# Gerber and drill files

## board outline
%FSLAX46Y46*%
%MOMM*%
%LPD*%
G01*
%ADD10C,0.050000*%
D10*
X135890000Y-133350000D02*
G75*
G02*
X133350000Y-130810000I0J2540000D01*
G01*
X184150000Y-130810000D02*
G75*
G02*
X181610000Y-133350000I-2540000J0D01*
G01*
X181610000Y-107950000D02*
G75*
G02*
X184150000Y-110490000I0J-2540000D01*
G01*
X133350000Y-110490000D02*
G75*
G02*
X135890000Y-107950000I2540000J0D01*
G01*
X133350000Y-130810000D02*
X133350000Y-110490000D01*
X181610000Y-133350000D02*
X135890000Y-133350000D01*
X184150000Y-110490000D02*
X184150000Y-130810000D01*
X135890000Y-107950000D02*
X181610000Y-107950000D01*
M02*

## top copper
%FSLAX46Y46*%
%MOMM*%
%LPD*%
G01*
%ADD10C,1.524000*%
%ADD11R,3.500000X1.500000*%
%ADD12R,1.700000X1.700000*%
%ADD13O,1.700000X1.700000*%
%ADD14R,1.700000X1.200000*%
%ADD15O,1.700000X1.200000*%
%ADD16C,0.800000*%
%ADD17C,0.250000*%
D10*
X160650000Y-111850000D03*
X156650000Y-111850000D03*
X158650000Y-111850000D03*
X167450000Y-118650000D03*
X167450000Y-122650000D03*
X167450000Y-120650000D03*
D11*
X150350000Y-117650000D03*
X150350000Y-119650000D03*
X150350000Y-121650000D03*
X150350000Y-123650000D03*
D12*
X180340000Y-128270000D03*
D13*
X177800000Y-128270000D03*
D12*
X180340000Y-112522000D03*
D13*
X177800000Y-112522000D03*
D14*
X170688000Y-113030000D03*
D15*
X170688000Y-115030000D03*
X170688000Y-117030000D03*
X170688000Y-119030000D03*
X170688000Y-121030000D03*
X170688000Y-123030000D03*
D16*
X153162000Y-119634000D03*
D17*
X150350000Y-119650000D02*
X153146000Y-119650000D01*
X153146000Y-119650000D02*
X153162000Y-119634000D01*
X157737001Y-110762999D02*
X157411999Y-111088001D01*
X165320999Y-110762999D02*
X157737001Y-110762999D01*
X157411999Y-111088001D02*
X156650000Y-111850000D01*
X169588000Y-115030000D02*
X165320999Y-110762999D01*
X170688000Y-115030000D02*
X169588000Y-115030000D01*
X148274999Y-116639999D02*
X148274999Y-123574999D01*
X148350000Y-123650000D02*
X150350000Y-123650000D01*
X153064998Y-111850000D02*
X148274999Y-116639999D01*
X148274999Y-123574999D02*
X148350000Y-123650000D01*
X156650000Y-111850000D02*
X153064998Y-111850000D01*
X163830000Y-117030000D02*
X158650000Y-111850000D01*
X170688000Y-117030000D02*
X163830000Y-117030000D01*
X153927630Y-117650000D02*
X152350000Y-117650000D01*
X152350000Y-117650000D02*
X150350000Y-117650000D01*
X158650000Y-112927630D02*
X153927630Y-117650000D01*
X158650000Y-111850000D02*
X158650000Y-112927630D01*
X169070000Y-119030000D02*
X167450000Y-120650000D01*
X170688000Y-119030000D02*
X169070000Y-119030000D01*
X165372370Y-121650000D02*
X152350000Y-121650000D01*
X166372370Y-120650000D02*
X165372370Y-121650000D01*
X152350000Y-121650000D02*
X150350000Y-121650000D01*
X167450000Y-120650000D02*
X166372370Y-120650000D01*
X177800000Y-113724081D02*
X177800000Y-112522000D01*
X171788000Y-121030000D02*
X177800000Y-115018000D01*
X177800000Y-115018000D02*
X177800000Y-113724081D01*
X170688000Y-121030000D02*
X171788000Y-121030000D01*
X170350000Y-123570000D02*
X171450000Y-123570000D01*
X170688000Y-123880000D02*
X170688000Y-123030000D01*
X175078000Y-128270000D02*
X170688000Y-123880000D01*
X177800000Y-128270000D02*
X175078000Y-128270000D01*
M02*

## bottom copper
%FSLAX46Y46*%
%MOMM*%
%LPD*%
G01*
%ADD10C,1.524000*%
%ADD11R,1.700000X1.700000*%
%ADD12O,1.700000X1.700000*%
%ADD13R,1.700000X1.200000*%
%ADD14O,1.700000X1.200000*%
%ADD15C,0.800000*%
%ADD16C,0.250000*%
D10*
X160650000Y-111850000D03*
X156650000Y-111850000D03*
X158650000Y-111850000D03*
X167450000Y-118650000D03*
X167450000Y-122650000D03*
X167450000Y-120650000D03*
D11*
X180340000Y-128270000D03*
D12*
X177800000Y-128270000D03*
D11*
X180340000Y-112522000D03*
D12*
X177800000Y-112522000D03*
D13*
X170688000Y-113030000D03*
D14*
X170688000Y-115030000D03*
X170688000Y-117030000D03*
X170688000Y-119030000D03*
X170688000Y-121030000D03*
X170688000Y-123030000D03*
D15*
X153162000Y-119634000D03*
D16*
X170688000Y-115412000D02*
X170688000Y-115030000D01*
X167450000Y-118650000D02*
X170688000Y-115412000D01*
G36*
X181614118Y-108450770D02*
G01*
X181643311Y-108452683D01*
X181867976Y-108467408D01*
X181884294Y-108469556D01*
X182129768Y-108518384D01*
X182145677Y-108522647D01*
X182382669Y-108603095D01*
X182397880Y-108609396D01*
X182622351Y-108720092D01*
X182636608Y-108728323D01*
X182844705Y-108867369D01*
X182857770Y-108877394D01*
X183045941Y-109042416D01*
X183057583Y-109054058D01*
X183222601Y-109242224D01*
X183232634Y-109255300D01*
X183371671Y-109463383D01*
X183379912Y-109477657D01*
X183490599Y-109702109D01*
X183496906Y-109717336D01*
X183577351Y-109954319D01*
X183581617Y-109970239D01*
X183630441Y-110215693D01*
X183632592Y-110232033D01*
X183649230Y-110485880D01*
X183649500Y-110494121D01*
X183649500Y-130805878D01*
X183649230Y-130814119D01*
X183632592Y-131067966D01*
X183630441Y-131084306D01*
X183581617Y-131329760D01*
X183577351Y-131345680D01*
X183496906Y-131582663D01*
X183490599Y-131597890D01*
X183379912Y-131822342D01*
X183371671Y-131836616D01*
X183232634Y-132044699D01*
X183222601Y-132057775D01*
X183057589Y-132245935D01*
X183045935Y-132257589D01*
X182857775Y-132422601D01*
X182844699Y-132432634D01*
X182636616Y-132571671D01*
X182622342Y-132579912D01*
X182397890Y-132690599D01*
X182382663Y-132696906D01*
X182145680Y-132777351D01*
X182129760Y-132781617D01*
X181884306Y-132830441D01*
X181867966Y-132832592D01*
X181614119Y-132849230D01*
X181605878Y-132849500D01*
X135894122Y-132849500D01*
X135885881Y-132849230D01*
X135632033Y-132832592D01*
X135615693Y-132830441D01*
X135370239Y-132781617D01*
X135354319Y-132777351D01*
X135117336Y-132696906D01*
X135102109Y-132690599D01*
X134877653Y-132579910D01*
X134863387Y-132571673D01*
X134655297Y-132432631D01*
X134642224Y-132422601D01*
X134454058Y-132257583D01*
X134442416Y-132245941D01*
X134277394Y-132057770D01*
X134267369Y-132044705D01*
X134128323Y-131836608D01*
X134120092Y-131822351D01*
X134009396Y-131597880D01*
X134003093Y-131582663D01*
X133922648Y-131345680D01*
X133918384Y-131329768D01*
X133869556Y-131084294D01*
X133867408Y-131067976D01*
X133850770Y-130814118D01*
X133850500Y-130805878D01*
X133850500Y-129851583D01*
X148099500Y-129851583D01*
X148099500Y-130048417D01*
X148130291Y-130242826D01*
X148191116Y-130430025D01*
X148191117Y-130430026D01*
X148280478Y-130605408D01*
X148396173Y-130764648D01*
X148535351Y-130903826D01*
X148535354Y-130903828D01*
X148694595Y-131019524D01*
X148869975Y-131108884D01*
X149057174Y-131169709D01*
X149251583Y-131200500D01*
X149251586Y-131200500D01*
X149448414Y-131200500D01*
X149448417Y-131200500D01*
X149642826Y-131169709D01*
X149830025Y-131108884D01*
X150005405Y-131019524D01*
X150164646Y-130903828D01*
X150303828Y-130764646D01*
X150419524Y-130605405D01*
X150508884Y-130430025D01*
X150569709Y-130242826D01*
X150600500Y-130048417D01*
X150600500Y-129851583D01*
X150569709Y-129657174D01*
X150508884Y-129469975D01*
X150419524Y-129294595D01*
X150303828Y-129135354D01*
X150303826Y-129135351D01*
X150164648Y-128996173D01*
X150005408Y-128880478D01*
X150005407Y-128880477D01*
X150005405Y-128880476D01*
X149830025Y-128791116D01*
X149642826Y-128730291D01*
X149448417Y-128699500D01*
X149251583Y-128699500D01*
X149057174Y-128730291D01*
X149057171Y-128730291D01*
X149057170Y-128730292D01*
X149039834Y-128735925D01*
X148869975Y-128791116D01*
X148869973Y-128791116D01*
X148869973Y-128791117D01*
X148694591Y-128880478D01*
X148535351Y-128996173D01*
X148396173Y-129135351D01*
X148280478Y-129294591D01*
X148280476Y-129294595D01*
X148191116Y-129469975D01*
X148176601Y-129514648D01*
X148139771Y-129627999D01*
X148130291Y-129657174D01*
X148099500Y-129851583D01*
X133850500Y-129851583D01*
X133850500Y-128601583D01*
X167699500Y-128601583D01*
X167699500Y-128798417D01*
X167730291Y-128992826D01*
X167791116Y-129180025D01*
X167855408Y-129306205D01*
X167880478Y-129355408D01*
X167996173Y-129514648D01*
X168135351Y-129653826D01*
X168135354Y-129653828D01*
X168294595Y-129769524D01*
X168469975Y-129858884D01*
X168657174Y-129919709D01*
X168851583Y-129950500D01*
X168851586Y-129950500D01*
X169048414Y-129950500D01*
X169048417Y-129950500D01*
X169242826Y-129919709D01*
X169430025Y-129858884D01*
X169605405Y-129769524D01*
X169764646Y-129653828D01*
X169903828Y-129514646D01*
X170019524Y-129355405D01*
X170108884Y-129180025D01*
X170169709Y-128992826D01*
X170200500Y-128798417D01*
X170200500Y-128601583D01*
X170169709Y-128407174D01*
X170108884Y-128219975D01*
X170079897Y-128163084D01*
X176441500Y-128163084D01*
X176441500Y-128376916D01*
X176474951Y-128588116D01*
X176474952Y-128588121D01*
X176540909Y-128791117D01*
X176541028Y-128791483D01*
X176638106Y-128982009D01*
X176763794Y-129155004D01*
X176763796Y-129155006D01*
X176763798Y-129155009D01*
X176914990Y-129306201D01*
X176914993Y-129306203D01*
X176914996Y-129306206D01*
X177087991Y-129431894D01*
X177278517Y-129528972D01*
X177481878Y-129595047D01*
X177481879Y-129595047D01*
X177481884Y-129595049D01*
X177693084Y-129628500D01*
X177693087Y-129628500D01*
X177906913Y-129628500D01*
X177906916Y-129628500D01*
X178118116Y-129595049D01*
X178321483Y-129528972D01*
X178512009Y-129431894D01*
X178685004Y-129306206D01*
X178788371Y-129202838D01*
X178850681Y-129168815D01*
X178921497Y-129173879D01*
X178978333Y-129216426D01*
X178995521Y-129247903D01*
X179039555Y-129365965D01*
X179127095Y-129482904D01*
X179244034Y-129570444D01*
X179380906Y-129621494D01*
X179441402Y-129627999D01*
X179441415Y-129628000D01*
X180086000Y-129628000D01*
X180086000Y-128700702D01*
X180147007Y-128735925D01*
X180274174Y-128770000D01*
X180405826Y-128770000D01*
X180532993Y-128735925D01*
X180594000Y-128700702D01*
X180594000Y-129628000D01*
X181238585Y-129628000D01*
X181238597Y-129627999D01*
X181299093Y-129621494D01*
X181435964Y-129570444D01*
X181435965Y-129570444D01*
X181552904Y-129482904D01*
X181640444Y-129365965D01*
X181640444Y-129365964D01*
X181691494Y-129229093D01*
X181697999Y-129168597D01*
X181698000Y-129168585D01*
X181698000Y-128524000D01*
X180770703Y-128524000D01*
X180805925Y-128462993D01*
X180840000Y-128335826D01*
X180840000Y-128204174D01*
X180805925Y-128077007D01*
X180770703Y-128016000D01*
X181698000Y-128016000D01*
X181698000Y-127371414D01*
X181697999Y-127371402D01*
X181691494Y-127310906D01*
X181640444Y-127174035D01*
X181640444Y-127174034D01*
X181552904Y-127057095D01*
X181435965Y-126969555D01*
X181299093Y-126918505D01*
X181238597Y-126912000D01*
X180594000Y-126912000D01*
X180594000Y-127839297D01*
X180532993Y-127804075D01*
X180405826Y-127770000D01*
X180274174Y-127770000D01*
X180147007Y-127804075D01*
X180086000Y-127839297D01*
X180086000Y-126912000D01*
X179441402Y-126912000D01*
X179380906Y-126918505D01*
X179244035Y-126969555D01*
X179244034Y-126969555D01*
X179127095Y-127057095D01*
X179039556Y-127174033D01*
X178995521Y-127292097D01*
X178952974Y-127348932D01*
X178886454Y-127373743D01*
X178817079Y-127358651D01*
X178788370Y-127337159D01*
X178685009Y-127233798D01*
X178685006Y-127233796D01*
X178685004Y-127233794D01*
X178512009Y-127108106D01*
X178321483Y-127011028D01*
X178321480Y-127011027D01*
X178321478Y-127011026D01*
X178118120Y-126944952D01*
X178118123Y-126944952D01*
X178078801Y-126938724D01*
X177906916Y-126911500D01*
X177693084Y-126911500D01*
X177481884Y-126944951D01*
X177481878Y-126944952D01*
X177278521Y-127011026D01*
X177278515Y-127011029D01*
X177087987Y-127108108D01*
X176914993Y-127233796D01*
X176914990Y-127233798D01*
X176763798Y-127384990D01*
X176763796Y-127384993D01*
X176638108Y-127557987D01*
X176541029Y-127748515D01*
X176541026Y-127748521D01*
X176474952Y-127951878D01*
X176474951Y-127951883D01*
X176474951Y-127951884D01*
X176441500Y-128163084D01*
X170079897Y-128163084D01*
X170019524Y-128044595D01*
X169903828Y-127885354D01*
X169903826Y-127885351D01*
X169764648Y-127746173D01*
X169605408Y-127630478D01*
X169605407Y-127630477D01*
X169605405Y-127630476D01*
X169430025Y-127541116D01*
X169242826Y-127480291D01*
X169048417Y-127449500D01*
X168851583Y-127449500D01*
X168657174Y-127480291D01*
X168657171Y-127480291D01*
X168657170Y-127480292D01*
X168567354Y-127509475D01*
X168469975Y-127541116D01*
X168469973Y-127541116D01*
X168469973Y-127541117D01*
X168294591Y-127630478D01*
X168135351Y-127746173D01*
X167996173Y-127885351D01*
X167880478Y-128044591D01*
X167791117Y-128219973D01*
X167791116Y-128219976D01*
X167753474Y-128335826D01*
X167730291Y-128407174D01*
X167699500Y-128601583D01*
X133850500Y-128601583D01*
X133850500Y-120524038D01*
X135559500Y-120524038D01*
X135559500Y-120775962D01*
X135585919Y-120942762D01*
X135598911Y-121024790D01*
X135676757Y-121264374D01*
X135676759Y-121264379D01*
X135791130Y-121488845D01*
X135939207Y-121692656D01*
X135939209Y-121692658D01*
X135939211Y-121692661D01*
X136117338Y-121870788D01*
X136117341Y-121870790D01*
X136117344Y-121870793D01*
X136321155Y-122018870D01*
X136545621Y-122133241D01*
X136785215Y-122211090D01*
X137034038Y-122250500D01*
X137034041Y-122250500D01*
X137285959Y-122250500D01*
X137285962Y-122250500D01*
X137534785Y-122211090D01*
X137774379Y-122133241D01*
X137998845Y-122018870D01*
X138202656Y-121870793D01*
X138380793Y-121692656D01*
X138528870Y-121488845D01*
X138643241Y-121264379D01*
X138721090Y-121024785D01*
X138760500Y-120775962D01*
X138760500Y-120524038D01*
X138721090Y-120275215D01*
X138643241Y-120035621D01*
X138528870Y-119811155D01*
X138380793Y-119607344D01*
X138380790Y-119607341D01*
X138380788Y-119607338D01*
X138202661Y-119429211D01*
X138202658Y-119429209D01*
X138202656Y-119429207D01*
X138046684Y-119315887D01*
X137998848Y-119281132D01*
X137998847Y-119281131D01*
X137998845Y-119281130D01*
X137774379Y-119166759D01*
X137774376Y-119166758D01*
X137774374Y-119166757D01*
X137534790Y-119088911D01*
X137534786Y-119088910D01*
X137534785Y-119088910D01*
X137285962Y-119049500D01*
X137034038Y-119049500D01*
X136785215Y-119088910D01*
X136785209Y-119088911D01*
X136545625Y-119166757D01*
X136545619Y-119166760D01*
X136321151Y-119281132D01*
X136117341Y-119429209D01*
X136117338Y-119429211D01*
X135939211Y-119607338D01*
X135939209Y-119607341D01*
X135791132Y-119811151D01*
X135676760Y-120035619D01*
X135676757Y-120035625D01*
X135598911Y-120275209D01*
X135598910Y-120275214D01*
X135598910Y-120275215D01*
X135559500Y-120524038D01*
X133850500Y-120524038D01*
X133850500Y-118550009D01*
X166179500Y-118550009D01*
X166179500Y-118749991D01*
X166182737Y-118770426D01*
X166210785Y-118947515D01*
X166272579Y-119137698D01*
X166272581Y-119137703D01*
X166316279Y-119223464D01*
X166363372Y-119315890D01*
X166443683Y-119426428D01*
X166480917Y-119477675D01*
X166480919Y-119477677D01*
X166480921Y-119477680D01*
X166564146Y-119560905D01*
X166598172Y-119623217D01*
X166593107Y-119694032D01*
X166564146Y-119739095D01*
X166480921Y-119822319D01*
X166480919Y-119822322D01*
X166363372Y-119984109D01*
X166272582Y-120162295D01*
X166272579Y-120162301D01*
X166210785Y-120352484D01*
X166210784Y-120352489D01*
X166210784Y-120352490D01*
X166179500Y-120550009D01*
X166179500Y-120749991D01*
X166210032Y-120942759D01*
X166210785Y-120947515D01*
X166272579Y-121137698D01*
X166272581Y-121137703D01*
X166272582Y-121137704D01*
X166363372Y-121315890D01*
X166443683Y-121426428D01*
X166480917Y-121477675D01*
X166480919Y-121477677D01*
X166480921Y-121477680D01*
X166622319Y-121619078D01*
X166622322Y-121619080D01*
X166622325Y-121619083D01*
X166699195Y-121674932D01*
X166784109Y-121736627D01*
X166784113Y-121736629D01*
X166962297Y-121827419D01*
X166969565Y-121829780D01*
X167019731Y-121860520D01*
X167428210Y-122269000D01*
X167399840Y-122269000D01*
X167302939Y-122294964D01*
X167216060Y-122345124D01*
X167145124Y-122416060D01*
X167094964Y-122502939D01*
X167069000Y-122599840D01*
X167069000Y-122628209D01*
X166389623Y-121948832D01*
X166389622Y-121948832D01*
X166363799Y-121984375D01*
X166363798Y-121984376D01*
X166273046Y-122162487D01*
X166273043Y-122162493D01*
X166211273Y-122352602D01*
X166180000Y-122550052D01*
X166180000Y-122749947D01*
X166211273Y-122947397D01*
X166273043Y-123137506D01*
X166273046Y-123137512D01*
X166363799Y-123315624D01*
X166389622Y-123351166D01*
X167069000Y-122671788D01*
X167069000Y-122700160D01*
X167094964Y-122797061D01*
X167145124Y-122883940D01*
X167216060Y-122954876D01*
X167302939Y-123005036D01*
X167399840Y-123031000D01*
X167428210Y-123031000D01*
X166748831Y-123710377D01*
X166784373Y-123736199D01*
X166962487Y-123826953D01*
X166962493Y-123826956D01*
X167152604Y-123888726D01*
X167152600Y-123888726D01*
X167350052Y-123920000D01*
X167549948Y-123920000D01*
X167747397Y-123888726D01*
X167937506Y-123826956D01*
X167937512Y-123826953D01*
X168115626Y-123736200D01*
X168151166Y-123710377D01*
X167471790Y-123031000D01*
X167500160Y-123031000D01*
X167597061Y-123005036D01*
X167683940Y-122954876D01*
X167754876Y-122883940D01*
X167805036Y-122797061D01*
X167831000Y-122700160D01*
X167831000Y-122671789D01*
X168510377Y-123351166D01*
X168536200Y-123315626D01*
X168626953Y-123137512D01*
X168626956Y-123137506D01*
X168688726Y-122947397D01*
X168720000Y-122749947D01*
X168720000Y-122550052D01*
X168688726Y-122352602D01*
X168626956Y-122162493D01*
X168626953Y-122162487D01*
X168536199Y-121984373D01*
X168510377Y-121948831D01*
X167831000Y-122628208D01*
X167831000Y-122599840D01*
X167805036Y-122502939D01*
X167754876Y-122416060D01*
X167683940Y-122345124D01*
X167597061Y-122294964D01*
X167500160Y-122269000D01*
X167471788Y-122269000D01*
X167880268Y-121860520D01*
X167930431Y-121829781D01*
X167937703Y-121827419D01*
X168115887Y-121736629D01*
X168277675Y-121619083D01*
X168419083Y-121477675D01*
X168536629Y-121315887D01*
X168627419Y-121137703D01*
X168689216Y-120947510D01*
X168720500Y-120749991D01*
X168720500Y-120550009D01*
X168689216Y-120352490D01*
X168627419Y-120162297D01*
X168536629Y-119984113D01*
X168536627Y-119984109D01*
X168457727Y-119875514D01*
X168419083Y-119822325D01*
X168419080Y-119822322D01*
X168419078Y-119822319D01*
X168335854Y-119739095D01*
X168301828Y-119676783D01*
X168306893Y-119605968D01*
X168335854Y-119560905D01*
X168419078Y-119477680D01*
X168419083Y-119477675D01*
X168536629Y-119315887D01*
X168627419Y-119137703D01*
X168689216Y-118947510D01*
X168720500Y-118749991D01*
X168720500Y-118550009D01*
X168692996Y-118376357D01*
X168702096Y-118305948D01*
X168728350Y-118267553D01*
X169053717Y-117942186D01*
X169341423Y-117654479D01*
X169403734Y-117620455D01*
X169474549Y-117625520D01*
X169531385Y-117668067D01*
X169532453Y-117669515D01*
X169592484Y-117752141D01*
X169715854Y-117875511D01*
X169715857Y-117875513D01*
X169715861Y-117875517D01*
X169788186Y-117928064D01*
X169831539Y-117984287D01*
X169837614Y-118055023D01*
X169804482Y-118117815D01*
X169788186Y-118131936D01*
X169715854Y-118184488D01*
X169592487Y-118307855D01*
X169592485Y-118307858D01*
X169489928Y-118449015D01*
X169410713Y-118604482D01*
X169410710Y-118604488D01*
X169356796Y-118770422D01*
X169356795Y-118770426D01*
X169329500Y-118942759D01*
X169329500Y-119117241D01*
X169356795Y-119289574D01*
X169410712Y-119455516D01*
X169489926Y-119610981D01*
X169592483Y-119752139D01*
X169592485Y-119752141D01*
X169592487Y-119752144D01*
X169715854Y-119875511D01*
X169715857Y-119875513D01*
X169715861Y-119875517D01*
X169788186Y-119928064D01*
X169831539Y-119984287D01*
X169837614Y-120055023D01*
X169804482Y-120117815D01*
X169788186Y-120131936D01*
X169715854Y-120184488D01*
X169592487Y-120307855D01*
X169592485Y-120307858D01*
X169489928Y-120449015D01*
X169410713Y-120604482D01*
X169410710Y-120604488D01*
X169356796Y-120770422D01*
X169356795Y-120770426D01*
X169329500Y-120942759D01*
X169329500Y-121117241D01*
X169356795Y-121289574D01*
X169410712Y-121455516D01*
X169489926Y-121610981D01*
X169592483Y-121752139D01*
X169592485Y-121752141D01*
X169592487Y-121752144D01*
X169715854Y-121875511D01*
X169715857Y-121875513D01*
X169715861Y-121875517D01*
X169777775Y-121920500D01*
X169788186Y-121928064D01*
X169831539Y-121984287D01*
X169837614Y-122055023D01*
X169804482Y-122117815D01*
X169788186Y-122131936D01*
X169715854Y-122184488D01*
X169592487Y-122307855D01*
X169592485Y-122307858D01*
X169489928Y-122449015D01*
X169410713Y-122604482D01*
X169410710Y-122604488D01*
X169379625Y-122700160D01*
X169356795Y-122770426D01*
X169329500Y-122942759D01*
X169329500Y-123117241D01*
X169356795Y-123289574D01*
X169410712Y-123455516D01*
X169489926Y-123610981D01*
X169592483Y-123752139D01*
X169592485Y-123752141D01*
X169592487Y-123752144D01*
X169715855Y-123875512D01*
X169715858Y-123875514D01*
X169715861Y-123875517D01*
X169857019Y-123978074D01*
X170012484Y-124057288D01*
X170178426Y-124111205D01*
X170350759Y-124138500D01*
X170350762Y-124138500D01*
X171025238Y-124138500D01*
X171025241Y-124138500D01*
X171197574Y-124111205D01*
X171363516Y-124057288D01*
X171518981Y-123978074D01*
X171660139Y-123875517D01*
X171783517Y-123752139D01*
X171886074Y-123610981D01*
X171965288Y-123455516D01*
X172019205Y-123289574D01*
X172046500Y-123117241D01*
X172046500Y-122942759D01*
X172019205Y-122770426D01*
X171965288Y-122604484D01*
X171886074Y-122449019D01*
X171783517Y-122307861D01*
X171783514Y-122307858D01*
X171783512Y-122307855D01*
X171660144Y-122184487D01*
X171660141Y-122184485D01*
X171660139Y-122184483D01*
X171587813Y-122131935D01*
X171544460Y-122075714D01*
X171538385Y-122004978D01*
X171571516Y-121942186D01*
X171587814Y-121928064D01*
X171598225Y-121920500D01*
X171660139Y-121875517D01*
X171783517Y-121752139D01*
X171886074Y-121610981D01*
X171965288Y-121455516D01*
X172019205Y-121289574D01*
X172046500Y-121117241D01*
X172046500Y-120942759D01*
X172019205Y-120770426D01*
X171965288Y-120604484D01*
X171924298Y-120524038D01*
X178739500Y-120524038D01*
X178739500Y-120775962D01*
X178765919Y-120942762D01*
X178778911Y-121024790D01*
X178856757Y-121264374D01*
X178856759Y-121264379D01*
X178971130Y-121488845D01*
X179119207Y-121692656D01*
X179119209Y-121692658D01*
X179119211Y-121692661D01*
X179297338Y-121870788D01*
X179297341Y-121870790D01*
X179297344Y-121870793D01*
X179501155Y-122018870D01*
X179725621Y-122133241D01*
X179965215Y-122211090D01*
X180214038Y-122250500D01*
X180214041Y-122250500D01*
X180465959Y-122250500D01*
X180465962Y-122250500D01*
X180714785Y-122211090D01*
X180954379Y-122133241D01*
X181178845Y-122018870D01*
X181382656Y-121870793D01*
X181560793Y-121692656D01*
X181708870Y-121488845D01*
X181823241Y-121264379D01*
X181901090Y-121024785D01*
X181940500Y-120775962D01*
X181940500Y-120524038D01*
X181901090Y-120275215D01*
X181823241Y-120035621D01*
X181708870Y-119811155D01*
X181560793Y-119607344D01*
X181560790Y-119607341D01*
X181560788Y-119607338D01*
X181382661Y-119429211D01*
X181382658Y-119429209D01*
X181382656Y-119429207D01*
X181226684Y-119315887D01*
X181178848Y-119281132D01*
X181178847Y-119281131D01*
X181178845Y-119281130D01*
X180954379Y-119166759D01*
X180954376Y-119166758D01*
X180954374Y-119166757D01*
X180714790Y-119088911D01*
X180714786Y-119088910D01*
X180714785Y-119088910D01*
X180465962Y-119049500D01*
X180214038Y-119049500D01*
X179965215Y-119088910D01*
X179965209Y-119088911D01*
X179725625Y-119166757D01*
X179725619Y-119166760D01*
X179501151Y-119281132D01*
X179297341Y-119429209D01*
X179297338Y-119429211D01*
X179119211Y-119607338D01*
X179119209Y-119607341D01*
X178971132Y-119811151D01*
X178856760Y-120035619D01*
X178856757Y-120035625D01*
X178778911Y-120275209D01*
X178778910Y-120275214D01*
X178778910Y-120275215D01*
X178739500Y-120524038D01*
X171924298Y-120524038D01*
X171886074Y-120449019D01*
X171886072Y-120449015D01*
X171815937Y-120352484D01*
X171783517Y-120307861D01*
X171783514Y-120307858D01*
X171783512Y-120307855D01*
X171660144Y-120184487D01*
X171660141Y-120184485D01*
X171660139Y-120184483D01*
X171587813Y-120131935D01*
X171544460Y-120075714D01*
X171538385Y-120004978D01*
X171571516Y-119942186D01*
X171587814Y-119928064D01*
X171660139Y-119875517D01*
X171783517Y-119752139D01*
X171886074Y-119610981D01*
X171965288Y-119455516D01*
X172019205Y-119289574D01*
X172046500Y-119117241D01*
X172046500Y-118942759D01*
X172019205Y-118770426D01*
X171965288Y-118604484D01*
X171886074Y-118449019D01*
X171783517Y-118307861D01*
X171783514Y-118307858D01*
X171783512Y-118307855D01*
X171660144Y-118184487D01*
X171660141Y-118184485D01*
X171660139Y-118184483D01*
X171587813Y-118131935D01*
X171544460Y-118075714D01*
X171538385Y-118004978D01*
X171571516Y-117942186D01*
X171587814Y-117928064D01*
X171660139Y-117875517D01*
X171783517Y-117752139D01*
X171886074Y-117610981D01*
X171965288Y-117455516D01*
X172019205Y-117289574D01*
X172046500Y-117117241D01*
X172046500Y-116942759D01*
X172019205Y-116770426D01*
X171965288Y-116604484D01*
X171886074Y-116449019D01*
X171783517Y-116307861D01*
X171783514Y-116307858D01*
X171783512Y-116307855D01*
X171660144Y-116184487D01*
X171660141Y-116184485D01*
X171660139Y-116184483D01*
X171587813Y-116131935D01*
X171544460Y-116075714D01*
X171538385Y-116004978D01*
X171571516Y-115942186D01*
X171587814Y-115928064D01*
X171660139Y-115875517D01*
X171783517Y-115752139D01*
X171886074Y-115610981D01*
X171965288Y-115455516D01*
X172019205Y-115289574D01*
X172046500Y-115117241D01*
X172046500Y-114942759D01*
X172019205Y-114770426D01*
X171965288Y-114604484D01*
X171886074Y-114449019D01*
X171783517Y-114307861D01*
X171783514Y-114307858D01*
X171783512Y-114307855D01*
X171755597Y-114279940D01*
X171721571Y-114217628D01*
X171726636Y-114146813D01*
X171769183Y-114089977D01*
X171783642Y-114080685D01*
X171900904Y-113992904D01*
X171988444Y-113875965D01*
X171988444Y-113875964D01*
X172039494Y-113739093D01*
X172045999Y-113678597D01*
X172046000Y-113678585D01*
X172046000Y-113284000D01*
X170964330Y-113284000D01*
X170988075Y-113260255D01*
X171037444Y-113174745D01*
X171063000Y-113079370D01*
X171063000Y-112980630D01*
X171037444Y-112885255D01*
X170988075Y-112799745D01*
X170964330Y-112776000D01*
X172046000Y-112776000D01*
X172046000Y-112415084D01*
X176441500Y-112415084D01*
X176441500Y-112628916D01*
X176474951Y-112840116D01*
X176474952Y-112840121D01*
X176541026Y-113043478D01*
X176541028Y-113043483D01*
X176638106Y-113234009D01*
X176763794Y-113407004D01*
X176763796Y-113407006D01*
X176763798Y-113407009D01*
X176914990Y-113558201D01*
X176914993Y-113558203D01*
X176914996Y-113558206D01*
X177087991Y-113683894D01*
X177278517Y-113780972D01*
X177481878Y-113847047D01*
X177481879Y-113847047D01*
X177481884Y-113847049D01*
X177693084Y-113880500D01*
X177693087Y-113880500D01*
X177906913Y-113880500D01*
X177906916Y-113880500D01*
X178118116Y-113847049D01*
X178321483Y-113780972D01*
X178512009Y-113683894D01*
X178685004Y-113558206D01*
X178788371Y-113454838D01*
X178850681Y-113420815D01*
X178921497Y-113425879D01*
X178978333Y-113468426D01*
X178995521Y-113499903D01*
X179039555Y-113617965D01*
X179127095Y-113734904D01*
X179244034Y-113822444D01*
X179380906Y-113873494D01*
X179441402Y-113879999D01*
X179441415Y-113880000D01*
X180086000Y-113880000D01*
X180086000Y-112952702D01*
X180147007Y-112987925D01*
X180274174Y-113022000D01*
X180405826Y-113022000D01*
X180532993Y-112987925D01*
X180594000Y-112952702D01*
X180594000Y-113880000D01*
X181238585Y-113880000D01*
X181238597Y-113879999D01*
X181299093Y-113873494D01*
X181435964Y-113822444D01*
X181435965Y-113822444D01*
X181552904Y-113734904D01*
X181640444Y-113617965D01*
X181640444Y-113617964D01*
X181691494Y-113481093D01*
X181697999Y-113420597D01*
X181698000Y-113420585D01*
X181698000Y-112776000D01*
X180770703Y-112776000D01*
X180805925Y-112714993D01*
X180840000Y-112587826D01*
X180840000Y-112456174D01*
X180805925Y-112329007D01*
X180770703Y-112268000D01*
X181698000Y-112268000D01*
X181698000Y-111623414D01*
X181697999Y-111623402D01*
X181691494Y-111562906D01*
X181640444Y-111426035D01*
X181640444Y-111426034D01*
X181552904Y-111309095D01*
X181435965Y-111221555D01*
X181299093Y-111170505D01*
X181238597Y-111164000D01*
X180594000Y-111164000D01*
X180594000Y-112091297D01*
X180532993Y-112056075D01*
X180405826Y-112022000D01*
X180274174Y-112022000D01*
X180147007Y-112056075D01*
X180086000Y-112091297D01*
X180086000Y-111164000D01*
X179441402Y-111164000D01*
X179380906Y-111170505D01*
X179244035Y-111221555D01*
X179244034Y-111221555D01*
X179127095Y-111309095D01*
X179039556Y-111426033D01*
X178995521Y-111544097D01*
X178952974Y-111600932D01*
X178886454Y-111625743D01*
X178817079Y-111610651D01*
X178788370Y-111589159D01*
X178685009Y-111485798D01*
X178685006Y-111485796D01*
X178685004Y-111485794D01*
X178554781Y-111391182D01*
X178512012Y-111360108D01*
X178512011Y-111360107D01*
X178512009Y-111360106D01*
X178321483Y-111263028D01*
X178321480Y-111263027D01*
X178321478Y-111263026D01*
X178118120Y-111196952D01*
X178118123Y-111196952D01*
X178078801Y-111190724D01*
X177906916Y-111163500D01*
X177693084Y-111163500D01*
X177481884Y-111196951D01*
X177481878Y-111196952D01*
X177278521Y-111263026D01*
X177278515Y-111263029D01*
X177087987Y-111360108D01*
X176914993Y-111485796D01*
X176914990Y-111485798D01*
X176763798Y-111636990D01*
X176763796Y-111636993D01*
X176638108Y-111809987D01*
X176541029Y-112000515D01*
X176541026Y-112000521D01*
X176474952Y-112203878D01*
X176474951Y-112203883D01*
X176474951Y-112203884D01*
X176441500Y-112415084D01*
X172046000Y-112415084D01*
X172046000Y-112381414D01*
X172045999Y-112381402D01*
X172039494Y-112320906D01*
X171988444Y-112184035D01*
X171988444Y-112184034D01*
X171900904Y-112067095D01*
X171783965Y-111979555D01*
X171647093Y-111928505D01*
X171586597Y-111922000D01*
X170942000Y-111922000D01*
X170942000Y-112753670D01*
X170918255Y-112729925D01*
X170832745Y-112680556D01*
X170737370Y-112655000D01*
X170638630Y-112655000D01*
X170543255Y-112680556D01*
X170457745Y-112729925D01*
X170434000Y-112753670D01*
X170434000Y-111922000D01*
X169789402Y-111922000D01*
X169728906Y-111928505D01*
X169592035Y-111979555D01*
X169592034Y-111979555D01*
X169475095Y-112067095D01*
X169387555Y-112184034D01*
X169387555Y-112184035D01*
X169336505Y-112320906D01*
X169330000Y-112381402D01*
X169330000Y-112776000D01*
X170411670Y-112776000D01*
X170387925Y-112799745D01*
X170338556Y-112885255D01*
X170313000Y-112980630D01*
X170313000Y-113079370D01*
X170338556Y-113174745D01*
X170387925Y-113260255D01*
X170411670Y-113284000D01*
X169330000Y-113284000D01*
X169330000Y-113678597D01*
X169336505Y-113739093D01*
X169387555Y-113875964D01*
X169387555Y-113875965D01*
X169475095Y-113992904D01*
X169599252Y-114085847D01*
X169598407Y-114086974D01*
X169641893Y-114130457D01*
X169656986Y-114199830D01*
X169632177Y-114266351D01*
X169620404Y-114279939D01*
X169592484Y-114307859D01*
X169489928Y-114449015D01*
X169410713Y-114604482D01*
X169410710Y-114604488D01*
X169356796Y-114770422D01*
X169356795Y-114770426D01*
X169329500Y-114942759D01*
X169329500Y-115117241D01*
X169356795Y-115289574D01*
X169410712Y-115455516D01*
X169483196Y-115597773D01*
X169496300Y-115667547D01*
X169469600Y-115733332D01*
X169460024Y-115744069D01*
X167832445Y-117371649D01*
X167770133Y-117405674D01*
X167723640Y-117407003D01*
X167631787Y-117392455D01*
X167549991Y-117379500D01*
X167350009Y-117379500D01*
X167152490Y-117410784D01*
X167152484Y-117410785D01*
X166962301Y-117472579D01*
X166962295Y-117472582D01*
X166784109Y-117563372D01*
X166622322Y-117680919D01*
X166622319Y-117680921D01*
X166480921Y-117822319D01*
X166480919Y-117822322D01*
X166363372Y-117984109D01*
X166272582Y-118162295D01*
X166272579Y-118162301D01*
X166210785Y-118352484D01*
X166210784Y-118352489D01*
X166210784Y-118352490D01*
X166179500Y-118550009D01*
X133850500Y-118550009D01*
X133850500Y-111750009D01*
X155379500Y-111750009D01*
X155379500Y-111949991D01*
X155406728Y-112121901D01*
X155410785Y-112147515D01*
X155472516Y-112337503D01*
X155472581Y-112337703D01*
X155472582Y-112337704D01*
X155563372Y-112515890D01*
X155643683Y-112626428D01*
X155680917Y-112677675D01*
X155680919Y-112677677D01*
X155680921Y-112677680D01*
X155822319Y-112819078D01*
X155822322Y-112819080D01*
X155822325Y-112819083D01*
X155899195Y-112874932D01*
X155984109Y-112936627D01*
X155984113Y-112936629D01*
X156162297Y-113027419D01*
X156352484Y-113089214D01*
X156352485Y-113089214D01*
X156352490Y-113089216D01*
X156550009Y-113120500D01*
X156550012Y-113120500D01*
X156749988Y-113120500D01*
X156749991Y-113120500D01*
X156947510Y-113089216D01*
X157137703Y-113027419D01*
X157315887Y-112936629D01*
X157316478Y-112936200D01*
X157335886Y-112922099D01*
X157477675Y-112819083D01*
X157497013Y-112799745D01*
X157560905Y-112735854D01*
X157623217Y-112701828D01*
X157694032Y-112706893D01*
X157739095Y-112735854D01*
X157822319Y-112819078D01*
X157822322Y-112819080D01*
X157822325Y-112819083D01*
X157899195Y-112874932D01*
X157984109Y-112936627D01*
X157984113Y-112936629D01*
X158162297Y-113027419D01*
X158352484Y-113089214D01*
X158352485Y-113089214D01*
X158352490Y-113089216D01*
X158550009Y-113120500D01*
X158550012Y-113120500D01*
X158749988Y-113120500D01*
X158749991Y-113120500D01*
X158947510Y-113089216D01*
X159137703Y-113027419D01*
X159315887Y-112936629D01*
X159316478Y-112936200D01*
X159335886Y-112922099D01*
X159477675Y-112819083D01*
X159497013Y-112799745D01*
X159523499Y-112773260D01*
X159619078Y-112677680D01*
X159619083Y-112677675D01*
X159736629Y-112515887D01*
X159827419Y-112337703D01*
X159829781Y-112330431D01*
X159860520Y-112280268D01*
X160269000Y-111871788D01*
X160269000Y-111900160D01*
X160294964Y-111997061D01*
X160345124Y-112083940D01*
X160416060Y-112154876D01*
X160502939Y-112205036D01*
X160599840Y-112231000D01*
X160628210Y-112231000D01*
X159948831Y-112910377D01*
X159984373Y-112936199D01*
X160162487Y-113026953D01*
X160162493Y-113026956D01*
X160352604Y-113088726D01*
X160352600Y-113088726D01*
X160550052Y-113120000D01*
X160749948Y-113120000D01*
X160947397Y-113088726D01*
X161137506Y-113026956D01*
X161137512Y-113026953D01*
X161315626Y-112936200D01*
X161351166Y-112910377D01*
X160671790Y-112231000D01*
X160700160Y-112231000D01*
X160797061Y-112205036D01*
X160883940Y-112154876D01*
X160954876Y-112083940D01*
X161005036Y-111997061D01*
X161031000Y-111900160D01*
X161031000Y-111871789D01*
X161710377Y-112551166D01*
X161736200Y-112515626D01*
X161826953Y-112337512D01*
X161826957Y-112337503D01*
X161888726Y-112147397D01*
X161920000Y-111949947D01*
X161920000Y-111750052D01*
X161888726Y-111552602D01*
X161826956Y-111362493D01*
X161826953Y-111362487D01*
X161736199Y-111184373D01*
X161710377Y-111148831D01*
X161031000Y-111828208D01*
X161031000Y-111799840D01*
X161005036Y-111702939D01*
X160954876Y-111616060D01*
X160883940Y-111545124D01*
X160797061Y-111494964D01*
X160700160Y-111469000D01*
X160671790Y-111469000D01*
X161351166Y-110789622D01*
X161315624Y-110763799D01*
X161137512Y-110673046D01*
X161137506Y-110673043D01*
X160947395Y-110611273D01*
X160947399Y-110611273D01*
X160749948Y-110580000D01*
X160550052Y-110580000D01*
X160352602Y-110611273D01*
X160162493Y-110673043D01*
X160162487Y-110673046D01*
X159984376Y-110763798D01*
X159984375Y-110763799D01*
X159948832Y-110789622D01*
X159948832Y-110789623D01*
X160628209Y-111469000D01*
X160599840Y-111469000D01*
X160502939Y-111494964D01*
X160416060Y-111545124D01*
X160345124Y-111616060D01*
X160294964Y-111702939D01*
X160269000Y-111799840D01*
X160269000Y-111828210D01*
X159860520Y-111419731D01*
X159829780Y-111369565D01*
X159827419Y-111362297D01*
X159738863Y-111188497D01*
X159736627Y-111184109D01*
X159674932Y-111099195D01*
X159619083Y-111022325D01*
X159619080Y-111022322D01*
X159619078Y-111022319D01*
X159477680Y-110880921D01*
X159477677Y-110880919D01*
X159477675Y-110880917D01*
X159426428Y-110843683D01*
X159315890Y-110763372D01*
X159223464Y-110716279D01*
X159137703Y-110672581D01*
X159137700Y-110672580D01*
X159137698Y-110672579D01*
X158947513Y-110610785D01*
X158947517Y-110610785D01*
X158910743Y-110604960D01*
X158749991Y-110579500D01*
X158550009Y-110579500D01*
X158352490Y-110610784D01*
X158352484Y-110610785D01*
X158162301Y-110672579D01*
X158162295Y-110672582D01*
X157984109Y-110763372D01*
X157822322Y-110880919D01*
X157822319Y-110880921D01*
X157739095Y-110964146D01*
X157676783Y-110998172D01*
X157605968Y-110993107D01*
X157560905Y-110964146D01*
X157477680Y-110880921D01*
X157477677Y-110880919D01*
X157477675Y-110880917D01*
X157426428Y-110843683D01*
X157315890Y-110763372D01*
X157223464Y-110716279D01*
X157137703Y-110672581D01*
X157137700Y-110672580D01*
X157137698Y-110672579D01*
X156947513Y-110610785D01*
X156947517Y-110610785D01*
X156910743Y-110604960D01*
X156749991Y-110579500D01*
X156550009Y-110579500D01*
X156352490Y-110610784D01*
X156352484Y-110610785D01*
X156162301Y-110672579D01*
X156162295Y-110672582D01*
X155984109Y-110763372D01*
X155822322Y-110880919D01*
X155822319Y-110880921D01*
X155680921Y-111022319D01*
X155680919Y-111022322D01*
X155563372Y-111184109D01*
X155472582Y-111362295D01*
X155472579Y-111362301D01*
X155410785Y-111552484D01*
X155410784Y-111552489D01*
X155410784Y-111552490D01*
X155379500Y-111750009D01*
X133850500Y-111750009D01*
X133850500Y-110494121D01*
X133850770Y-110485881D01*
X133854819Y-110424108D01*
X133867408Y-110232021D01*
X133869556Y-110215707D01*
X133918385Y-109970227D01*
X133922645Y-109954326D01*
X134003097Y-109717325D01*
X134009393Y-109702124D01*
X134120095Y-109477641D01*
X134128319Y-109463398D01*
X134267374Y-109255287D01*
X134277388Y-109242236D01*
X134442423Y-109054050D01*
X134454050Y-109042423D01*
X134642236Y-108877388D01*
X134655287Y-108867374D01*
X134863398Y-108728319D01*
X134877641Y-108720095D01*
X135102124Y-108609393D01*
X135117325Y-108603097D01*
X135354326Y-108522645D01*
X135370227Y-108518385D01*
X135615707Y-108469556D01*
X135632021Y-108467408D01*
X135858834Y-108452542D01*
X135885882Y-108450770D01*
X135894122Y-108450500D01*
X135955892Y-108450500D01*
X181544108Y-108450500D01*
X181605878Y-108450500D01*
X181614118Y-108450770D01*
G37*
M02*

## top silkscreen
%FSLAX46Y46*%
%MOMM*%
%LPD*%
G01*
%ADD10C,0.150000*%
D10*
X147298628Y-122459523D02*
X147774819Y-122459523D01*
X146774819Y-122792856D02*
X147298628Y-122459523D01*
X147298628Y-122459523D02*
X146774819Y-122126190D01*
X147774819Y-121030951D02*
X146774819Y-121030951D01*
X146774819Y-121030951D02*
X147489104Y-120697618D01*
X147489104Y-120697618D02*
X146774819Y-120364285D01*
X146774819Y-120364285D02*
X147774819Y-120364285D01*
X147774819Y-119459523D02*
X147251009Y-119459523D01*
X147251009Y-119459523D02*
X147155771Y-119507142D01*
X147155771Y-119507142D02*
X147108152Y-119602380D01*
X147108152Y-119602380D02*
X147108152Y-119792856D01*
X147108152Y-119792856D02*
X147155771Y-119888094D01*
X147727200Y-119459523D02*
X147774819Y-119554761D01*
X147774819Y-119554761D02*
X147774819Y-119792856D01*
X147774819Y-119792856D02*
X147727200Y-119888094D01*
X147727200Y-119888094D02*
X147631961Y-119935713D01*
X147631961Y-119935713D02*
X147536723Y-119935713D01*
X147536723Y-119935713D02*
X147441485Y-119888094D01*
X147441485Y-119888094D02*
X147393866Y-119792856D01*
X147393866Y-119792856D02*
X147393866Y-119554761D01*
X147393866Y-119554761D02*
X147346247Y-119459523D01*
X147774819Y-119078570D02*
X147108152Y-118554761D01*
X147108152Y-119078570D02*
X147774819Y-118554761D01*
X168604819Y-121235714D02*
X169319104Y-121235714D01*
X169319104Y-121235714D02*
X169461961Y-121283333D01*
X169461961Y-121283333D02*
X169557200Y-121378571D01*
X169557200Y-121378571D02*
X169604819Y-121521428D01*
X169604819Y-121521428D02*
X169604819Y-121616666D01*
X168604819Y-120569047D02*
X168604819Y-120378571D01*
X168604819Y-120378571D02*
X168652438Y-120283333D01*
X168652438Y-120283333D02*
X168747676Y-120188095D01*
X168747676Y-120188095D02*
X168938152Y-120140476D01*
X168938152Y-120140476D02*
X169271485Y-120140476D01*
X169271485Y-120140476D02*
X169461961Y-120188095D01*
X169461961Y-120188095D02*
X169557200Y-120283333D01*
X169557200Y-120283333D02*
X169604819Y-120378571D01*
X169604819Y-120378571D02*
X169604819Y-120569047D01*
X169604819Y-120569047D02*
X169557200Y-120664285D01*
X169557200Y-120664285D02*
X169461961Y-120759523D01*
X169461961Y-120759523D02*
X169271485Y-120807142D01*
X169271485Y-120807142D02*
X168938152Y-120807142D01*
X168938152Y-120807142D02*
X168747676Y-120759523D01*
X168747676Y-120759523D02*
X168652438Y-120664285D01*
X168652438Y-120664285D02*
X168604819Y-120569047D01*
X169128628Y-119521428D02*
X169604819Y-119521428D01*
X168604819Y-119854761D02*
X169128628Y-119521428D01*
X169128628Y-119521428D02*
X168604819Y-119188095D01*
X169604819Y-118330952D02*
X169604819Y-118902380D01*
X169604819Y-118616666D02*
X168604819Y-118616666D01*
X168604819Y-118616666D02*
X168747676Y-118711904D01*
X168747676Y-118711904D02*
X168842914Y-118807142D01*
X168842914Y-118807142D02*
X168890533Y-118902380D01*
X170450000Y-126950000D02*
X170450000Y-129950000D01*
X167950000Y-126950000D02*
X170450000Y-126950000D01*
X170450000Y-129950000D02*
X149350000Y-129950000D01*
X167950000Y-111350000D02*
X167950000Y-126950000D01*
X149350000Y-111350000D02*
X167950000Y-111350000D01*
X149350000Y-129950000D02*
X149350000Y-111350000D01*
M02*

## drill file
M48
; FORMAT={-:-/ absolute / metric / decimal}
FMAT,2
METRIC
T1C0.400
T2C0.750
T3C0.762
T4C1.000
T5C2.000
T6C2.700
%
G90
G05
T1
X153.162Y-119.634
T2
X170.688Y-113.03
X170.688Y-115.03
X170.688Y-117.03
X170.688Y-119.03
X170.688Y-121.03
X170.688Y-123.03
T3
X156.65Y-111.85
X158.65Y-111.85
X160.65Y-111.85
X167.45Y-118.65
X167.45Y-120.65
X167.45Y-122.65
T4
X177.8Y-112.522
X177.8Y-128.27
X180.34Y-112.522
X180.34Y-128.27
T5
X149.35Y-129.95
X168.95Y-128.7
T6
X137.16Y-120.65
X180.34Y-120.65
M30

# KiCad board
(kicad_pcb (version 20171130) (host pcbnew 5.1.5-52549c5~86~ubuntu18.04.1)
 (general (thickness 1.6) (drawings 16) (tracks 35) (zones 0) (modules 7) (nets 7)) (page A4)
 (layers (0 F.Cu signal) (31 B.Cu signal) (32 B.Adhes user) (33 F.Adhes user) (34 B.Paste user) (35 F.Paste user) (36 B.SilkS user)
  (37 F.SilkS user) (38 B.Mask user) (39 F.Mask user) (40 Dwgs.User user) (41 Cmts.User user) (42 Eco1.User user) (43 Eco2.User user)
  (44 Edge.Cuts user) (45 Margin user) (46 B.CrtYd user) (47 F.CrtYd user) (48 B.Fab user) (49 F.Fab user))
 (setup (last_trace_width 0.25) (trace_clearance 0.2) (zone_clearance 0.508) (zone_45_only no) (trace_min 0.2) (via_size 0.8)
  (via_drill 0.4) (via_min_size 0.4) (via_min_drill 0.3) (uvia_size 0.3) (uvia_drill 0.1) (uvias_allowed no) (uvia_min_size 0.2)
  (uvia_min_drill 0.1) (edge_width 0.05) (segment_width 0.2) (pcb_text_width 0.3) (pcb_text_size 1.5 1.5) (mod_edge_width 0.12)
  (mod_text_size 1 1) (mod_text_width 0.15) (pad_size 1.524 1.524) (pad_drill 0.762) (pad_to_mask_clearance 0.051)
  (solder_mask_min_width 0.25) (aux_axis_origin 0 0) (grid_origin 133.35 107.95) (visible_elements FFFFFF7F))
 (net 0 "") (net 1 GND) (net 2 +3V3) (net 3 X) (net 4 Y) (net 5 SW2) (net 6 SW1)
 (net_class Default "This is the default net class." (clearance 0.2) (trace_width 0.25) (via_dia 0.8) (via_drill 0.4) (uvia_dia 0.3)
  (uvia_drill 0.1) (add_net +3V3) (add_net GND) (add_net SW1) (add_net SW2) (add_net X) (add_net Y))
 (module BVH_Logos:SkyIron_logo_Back (layer F.Cu) (at 146.558 125.984)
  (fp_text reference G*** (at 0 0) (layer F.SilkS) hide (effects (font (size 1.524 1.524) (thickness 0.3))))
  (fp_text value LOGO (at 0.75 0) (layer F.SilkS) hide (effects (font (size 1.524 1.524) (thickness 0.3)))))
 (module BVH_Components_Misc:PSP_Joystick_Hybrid (layer F.Cu) (at 158.75 120.65 90)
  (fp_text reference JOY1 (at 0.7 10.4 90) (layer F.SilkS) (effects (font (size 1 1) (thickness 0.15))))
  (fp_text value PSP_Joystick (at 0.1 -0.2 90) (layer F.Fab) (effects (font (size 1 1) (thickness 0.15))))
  (fp_line (start -6.3 11.7) (end -9.3 11.7) (layer F.SilkS) (width 0.15))
  (fp_line (start -6.3 9.2) (end -6.3 11.7) (layer F.SilkS) (width 0.15))
  (fp_line (start -9.3 11.7) (end -9.3 -9.4) (layer F.SilkS) (width 0.15))
  (fp_line (start 9.3 9.2) (end -6.3 9.2) (layer F.SilkS) (width 0.15))
  (fp_line (start 9.3 -9.4) (end 9.3 9.2) (layer F.SilkS) (width 0.15))
  (fp_line (start -9.3 -9.4) (end 9.3 -9.4) (layer F.SilkS) (width 0.15))
  (pad 3 thru_hole circle (at 8.8 1.9 180) (size 1.524 1.524) (drill 0.762) (layers *.Cu *.Mask) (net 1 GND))
  (pad 1 thru_hole circle (at 8.8 -2.1 180) (size 1.524 1.524) (drill 0.762) (layers *.Cu *.Mask) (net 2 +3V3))
  (pad 4 thru_hole circle (at 8.8 -0.1 180) (size 1.524 1.524) (drill 0.762) (layers *.Cu *.Mask) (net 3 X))
  (pad 1 thru_hole circle (at 2 8.7 90) (size 1.524 1.524) (drill 0.762) (layers *.Cu *.Mask) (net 2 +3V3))
  (pad 3 thru_hole circle (at -2 8.7 90) (size 1.524 1.524) (drill 0.762) (layers *.Cu *.Mask) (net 1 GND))
  (pad 2 thru_hole circle (at 0 8.7 90) (size 1.524 1.524) (drill 0.762) (layers *.Cu *.Mask) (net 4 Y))
  (pad "" np_thru_hole circle (at -8.05 10.2 90) (size 2 2) (drill 2) (layers *.Cu *.Mask))
  (pad "" np_thru_hole circle (at -9.3 -9.4 90) (size 2 2) (drill 2) (layers *.Cu *.Mask))
  (pad 4 smd rect (at 3 -8.4 90) (size 1.5 3.5) (layers F.Cu F.Paste F.Mask) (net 3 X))
  (pad 3 smd rect (at 1 -8.4 90) (size 1.5 3.5) (layers F.Cu F.Paste F.Mask) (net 1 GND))
  (pad 2 smd rect (at -1 -8.4 90) (size 1.5 3.5) (layers F.Cu F.Paste F.Mask) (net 4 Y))
  (pad 1 smd rect (at -3 -8.4 90) (size 1.5 3.5) (layers F.Cu F.Paste F.Mask) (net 2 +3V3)))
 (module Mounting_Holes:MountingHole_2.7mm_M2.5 (layer F.Cu) (at 137.16 120.65)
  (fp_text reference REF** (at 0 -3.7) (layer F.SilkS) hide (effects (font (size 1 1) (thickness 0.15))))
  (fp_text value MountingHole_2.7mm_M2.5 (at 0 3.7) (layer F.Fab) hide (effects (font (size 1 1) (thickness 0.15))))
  (pad 1 np_thru_hole circle (at 0 0) (size 2.7 2.7) (drill 2.7) (layers *.Cu *.Mask)))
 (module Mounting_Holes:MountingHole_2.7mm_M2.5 (layer F.Cu) (at 180.34 120.65)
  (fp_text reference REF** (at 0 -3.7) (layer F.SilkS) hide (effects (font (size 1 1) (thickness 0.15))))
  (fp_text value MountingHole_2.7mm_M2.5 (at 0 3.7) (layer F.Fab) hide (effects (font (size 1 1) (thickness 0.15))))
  (pad 1 np_thru_hole circle (at 0 0) (size 2.7 2.7) (drill 2.7) (layers *.Cu *.Mask)))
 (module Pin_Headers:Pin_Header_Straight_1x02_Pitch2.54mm (layer B.Cu) (at 180.34 128.27 90)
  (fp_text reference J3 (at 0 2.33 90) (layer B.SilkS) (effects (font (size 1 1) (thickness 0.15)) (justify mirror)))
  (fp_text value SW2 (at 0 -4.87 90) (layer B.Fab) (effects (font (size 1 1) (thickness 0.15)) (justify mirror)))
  (pad 1 thru_hole rect (at 0 0 90) (size 1.7 1.7) (drill 1) (layers *.Cu *.Mask) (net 1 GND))
  (pad 2 thru_hole oval (at 0 -2.54 90) (size 1.7 1.7) (drill 1) (layers *.Cu *.Mask) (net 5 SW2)))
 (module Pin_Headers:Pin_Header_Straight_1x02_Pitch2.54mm (layer B.Cu) (at 180.34 112.522 90)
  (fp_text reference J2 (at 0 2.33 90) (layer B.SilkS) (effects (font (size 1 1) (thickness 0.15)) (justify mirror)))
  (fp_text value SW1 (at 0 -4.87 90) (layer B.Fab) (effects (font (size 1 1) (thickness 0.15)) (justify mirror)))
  (pad 1 thru_hole rect (at 0 0 90) (size 1.7 1.7) (drill 1) (layers *.Cu *.Mask) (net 1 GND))
  (pad 2 thru_hole oval (at 0 -2.54 90) (size 1.7 1.7) (drill 1) (layers *.Cu *.Mask) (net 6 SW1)))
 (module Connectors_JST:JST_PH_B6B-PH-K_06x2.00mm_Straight (layer B.Cu) (at 170.688 113.03 270)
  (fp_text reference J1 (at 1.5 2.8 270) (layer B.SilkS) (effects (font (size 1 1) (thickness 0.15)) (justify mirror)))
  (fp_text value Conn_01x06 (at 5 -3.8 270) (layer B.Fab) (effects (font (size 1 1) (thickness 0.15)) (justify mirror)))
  (pad 1 thru_hole rect (at 0 0 270) (size 1.2 1.7) (drill 0.75) (layers *.Cu *.Mask) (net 1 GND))
  (pad 2 thru_hole oval (at 2 0 270) (size 1.2 1.7) (drill 0.75) (layers *.Cu *.Mask) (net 2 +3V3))
  (pad 3 thru_hole oval (at 4 0 270) (size 1.2 1.7) (drill 0.75) (layers *.Cu *.Mask) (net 3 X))
  (pad 4 thru_hole oval (at 6 0 270) (size 1.2 1.7) (drill 0.75) (layers *.Cu *.Mask) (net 4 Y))
  (pad 5 thru_hole oval (at 8 0 270) (size 1.2 1.7) (drill 0.75) (layers *.Cu *.Mask) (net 6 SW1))
  (pad 6 thru_hole oval (at 10 0 270) (size 1.2 1.7) (drill 0.75) (layers *.Cu *.Mask) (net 5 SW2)))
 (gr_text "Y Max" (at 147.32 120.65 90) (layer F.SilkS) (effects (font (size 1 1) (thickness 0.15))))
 (gr_arc (start 135.89 130.81) (end 133.35 130.81) (angle -90) (layer Edge.Cuts) (width 0.05))
 (gr_arc (start 181.61 130.81) (end 181.61 133.35) (angle -90) (layer Edge.Cuts) (width 0.05))
 (gr_arc (start 181.61 110.49) (end 184.15 110.49) (angle -90) (layer Edge.Cuts) (width 0.05))
 (gr_arc (start 135.89 110.49) (end 135.89 107.95) (angle -90) (layer Edge.Cuts) (width 0.05))
 (gr_line (start 133.35 130.81) (end 133.35 110.49) (layer Edge.Cuts) (width 0.05))
 (gr_line (start 181.61 133.35) (end 135.89 133.35) (layer Edge.Cuts) (width 0.05))
 (gr_line (start 184.15 110.49) (end 184.15 130.81) (layer Edge.Cuts) (width 0.05))
 (gr_line (start 135.89 107.95) (end 181.61 107.95) (layer Edge.Cuts) (width 0.05))
 (via (at 153.162 119.634) (size 0.8) (drill 0.4) (layers F.Cu B.Cu) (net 1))
 (segment (start 150.35 119.65) (end 153.146 119.65) (width 0.25) (layer F.Cu) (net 1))
 (segment (start 153.146 119.65) (end 153.162 119.634) (width 0.25) (layer F.Cu) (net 1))
 (segment (start 170.688 115.412) (end 170.688 115.03) (width 0.25) (layer B.Cu) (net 2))
 (segment (start 167.45 118.65) (end 170.688 115.412) (width 0.25) (layer B.Cu) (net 2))
 (segment (start 157.737001 110.762999) (end 157.411999 111.088001) (width 0.25) (layer F.Cu) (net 2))
 (segment (start 165.320999 110.762999) (end 157.737001 110.762999) (width 0.25) (layer F.Cu) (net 2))
 (segment (start 157.411999 111.088001) (end 156.65 111.85) (width 0.25) (layer F.Cu) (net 2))
 (segment (start 169.588 115.03) (end 165.320999 110.762999) (width 0.25) (layer F.Cu) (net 2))
 (segment (start 170.688 115.03) (end 169.588 115.03) (width 0.25) (layer F.Cu) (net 2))
 (segment (start 148.274999 116.639999) (end 148.274999 123.574999) (width 0.25) (layer F.Cu) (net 2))
 (segment (start 148.35 123.65) (end 150.35 123.65) (width 0.25) (layer F.Cu) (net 2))
 (segment (start 153.064998 111.85) (end 148.274999 116.639999) (width 0.25) (layer F.Cu) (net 2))
 (segment (start 148.274999 123.574999) (end 148.35 123.65) (width 0.25) (layer F.Cu) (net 2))
 (segment (start 156.65 111.85) (end 153.064998 111.85) (width 0.25) (layer F.Cu) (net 2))
 (segment (start 163.83 117.03) (end 158.65 111.85) (width 0.25) (layer F.Cu) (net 3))
 (segment (start 170.688 117.03) (end 163.83 117.03) (width 0.25) (layer F.Cu) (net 3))
 (segment (start 153.92763 117.65) (end 152.35 117.65) (width 0.25) (layer F.Cu) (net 3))
 (segment (start 152.35 117.65) (end 150.35 117.65) (width 0.25) (layer F.Cu) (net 3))
 (segment (start 158.65 112.92763) (end 153.92763 117.65) (width 0.25) (layer F.Cu) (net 3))
 (segment (start 158.65 111.85) (end 158.65 112.92763) (width 0.25) (layer F.Cu) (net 3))
 (segment (start 169.07 119.03) (end 167.45 120.65) (width 0.25) (layer F.Cu) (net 4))
 (segment (start 170.688 119.03) (end 169.07 119.03) (width 0.25) (layer F.Cu) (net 4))
 (segment (start 165.37237 121.65) (end 152.35 121.65) (width 0.25) (layer F.Cu) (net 4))
 (segment (start 166.37237 120.65) (end 165.37237 121.65) (width 0.25) (layer F.Cu) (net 4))
 (segment (start 152.35 121.65) (end 150.35 121.65) (width 0.25) (layer F.Cu) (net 4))
 (segment (start 167.45 120.65) (end 166.37237 120.65) (width 0.25) (layer F.Cu) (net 4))
 (segment (start 177.8 113.724081) (end 177.8 112.522) (width 0.25) (layer F.Cu) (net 6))
 (segment (start 171.788 121.03) (end 177.8 115.018) (width 0.25) (layer F.Cu) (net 6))
 (segment (start 177.8 115.018) (end 177.8 113.724081) (width 0.25) (layer F.Cu) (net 6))
 (segment (start 170.688 121.03) (end 171.788 121.03) (width 0.25) (layer F.Cu) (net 6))
 (segment (start 170.35 123.57) (end 171.45 123.57) (width 0.25) (layer F.Cu) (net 5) (status 20))
 (segment (start 170.688 123.88) (end 170.688 123.03) (width 0.25) (layer F.Cu) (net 5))
 (segment (start 175.078 128.27) (end 170.688 123.88) (width 0.25) (layer F.Cu) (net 5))
 (segment (start 177.8 128.27) (end 175.078 128.27) (width 0.25) (layer F.Cu) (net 5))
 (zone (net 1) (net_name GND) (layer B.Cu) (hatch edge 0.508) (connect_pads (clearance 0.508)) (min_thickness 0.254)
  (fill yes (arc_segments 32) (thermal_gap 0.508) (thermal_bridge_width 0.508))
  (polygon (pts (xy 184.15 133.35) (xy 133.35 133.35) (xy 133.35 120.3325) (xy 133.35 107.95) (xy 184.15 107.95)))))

